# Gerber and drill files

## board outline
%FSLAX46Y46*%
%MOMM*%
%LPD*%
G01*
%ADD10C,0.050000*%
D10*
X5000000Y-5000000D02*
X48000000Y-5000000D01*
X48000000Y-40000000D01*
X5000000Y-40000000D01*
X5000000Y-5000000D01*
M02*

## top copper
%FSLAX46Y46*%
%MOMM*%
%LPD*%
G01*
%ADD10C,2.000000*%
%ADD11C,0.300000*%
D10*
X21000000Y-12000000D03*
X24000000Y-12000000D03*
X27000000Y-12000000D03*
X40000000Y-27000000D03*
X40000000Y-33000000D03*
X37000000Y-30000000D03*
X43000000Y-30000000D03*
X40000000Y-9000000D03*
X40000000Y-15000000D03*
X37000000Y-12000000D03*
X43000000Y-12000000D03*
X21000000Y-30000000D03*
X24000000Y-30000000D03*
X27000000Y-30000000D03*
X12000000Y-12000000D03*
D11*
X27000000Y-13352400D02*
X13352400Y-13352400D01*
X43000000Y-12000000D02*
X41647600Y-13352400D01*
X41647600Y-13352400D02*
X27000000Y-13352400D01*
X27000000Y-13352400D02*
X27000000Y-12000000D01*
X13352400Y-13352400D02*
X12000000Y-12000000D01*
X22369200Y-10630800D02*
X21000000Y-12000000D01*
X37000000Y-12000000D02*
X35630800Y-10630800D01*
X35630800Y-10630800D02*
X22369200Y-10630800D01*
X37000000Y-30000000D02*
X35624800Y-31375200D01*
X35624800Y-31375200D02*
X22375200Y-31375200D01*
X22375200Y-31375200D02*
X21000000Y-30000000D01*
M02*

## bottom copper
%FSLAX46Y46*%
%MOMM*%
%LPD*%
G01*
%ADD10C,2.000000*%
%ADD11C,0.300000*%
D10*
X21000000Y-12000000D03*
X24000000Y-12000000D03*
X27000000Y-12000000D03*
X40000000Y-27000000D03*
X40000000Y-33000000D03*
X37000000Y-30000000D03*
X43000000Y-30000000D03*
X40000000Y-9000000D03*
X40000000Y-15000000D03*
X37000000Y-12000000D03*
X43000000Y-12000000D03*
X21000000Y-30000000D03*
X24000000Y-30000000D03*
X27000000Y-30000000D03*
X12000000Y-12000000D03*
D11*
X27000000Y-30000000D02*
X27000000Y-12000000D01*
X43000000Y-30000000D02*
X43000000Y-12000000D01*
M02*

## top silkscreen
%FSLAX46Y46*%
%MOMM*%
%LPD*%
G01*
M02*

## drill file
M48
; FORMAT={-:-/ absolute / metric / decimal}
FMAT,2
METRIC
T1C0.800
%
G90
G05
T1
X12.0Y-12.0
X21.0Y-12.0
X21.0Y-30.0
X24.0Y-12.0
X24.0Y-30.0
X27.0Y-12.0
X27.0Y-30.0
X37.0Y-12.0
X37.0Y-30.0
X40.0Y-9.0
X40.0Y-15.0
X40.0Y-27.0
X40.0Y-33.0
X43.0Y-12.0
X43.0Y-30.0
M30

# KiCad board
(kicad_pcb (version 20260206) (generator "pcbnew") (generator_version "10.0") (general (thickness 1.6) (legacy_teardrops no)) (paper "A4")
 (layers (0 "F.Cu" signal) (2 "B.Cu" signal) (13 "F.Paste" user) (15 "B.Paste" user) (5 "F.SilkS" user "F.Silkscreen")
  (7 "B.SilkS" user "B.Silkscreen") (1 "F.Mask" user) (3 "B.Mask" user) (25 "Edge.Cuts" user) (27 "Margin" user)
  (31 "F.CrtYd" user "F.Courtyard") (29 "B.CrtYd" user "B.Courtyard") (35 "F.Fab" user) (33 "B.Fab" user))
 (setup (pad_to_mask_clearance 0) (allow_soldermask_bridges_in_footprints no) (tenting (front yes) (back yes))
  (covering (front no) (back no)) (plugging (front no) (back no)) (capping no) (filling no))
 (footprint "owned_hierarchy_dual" (layer "F.Cu") (at 24 12)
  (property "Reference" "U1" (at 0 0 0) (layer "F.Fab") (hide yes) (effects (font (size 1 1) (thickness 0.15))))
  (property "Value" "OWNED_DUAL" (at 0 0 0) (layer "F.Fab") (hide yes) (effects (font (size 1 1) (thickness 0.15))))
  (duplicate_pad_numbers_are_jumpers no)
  (pad "1" thru_hole circle (at -3 0) (size 2 2) (drill 0.8) (layers "*.Cu" "*.Mask") (remove_unused_layers no) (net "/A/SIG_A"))
  (pad "2" thru_hole circle (at 0 0) (size 2 2) (drill 0.8) (layers "*.Cu" "*.Mask") (remove_unused_layers no) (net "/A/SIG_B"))
  (pad "3" thru_hole circle (at 3 0) (size 2 2) (drill 0.8) (layers "*.Cu" "*.Mask") (remove_unused_layers no) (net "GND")))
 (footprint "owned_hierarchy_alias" (layer "F.Cu") (at 40 30)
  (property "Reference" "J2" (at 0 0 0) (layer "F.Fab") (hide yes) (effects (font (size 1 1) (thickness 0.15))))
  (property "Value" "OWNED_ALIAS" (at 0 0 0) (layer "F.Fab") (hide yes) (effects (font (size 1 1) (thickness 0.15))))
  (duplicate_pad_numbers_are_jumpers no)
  (pad "MP" thru_hole circle (at 0 -3) (size 2 2) (drill 0.8) (layers "*.Cu" "*.Mask") (remove_unused_layers no))
  (pad "MP" thru_hole circle (at 0 3) (size 2 2) (drill 0.8) (layers "*.Cu" "*.Mask") (remove_unused_layers no))
  (pad "R" thru_hole circle (at -3 0) (size 2 2) (drill 0.8) (layers "*.Cu" "*.Mask") (remove_unused_layers no) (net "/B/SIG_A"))
  (pad "T" thru_hole circle (at 3 0) (size 2 2) (drill 0.8) (layers "*.Cu" "*.Mask") (remove_unused_layers no) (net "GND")))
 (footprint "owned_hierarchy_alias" (layer "F.Cu") (at 40 12)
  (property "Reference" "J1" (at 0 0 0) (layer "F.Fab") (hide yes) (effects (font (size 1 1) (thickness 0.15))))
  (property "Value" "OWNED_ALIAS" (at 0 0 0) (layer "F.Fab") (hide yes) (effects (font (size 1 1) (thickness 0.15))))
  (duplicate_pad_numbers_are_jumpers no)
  (pad "MP" thru_hole circle (at 0 -3) (size 2 2) (drill 0.8) (layers "*.Cu" "*.Mask") (remove_unused_layers no))
  (pad "MP" thru_hole circle (at 0 3) (size 2 2) (drill 0.8) (layers "*.Cu" "*.Mask") (remove_unused_layers no))
  (pad "R" thru_hole circle (at -3 0) (size 2 2) (drill 0.8) (layers "*.Cu" "*.Mask") (remove_unused_layers no) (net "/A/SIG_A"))
  (pad "T" thru_hole circle (at 3 0) (size 2 2) (drill 0.8) (layers "*.Cu" "*.Mask") (remove_unused_layers no) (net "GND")))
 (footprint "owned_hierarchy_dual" (layer "F.Cu") (at 24 30)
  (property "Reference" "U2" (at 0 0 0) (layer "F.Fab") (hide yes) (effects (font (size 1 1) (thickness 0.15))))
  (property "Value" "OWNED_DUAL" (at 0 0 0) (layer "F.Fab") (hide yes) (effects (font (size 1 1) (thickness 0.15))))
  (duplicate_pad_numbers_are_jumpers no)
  (pad "1" thru_hole circle (at -3 0) (size 2 2) (drill 0.8) (layers "*.Cu" "*.Mask") (remove_unused_layers no) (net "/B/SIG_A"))
  (pad "2" thru_hole circle (at 0 0) (size 2 2) (drill 0.8) (layers "*.Cu" "*.Mask") (remove_unused_layers no) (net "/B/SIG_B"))
  (pad "3" thru_hole circle (at 3 0) (size 2 2) (drill 0.8) (layers "*.Cu" "*.Mask") (remove_unused_layers no) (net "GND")))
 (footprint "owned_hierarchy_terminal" (layer "F.Cu") (at 12 12)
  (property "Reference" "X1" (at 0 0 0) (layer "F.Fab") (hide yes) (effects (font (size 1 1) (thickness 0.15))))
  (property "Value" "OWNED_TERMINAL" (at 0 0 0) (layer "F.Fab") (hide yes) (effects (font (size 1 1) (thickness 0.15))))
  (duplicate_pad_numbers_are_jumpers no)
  (pad "1" thru_hole circle (at 0 0) (size 2 2) (drill 0.8) (layers "*.Cu" "*.Mask") (remove_unused_layers no) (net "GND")))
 (gr_rect (start 5 5) (end 48 40) (stroke (width 0.05) (type default)) (fill no) (layer "Edge.Cuts"))
 (segment (start 27 13.3524) (end 13.3524 13.3524) (width 0.3) (layer "F.Cu") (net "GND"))
 (segment (start 43 12) (end 41.6476 13.3524) (width 0.3) (layer "F.Cu") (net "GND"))
 (segment (start 41.6476 13.3524) (end 27 13.3524) (width 0.3) (layer "F.Cu") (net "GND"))
 (segment (start 27 13.3524) (end 27 12) (width 0.3) (layer "F.Cu") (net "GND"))
 (segment (start 13.3524 13.3524) (end 12 12) (width 0.3) (layer "F.Cu") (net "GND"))
 (segment (start 27 30) (end 27 12) (width 0.3) (layer "B.Cu") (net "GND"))
 (segment (start 43 30) (end 43 12) (width 0.3) (layer "B.Cu") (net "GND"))
 (segment (start 22.3692 10.6308) (end 21 12) (width 0.3) (layer "F.Cu") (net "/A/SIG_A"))
 (segment (start 37 12) (end 35.6308 10.6308) (width 0.3) (layer "F.Cu") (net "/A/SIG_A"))
 (segment (start 35.6308 10.6308) (end 22.3692 10.6308) (width 0.3) (layer "F.Cu") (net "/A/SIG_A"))
 (segment (start 37 30) (end 35.6248 31.3752) (width 0.3) (layer "F.Cu") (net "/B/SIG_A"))
 (segment (start 35.6248 31.3752) (end 22.3752 31.3752) (width 0.3) (layer "F.Cu") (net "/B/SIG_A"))
 (segment (start 22.3752 31.3752) (end 21 30) (width 0.3) (layer "F.Cu") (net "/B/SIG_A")))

